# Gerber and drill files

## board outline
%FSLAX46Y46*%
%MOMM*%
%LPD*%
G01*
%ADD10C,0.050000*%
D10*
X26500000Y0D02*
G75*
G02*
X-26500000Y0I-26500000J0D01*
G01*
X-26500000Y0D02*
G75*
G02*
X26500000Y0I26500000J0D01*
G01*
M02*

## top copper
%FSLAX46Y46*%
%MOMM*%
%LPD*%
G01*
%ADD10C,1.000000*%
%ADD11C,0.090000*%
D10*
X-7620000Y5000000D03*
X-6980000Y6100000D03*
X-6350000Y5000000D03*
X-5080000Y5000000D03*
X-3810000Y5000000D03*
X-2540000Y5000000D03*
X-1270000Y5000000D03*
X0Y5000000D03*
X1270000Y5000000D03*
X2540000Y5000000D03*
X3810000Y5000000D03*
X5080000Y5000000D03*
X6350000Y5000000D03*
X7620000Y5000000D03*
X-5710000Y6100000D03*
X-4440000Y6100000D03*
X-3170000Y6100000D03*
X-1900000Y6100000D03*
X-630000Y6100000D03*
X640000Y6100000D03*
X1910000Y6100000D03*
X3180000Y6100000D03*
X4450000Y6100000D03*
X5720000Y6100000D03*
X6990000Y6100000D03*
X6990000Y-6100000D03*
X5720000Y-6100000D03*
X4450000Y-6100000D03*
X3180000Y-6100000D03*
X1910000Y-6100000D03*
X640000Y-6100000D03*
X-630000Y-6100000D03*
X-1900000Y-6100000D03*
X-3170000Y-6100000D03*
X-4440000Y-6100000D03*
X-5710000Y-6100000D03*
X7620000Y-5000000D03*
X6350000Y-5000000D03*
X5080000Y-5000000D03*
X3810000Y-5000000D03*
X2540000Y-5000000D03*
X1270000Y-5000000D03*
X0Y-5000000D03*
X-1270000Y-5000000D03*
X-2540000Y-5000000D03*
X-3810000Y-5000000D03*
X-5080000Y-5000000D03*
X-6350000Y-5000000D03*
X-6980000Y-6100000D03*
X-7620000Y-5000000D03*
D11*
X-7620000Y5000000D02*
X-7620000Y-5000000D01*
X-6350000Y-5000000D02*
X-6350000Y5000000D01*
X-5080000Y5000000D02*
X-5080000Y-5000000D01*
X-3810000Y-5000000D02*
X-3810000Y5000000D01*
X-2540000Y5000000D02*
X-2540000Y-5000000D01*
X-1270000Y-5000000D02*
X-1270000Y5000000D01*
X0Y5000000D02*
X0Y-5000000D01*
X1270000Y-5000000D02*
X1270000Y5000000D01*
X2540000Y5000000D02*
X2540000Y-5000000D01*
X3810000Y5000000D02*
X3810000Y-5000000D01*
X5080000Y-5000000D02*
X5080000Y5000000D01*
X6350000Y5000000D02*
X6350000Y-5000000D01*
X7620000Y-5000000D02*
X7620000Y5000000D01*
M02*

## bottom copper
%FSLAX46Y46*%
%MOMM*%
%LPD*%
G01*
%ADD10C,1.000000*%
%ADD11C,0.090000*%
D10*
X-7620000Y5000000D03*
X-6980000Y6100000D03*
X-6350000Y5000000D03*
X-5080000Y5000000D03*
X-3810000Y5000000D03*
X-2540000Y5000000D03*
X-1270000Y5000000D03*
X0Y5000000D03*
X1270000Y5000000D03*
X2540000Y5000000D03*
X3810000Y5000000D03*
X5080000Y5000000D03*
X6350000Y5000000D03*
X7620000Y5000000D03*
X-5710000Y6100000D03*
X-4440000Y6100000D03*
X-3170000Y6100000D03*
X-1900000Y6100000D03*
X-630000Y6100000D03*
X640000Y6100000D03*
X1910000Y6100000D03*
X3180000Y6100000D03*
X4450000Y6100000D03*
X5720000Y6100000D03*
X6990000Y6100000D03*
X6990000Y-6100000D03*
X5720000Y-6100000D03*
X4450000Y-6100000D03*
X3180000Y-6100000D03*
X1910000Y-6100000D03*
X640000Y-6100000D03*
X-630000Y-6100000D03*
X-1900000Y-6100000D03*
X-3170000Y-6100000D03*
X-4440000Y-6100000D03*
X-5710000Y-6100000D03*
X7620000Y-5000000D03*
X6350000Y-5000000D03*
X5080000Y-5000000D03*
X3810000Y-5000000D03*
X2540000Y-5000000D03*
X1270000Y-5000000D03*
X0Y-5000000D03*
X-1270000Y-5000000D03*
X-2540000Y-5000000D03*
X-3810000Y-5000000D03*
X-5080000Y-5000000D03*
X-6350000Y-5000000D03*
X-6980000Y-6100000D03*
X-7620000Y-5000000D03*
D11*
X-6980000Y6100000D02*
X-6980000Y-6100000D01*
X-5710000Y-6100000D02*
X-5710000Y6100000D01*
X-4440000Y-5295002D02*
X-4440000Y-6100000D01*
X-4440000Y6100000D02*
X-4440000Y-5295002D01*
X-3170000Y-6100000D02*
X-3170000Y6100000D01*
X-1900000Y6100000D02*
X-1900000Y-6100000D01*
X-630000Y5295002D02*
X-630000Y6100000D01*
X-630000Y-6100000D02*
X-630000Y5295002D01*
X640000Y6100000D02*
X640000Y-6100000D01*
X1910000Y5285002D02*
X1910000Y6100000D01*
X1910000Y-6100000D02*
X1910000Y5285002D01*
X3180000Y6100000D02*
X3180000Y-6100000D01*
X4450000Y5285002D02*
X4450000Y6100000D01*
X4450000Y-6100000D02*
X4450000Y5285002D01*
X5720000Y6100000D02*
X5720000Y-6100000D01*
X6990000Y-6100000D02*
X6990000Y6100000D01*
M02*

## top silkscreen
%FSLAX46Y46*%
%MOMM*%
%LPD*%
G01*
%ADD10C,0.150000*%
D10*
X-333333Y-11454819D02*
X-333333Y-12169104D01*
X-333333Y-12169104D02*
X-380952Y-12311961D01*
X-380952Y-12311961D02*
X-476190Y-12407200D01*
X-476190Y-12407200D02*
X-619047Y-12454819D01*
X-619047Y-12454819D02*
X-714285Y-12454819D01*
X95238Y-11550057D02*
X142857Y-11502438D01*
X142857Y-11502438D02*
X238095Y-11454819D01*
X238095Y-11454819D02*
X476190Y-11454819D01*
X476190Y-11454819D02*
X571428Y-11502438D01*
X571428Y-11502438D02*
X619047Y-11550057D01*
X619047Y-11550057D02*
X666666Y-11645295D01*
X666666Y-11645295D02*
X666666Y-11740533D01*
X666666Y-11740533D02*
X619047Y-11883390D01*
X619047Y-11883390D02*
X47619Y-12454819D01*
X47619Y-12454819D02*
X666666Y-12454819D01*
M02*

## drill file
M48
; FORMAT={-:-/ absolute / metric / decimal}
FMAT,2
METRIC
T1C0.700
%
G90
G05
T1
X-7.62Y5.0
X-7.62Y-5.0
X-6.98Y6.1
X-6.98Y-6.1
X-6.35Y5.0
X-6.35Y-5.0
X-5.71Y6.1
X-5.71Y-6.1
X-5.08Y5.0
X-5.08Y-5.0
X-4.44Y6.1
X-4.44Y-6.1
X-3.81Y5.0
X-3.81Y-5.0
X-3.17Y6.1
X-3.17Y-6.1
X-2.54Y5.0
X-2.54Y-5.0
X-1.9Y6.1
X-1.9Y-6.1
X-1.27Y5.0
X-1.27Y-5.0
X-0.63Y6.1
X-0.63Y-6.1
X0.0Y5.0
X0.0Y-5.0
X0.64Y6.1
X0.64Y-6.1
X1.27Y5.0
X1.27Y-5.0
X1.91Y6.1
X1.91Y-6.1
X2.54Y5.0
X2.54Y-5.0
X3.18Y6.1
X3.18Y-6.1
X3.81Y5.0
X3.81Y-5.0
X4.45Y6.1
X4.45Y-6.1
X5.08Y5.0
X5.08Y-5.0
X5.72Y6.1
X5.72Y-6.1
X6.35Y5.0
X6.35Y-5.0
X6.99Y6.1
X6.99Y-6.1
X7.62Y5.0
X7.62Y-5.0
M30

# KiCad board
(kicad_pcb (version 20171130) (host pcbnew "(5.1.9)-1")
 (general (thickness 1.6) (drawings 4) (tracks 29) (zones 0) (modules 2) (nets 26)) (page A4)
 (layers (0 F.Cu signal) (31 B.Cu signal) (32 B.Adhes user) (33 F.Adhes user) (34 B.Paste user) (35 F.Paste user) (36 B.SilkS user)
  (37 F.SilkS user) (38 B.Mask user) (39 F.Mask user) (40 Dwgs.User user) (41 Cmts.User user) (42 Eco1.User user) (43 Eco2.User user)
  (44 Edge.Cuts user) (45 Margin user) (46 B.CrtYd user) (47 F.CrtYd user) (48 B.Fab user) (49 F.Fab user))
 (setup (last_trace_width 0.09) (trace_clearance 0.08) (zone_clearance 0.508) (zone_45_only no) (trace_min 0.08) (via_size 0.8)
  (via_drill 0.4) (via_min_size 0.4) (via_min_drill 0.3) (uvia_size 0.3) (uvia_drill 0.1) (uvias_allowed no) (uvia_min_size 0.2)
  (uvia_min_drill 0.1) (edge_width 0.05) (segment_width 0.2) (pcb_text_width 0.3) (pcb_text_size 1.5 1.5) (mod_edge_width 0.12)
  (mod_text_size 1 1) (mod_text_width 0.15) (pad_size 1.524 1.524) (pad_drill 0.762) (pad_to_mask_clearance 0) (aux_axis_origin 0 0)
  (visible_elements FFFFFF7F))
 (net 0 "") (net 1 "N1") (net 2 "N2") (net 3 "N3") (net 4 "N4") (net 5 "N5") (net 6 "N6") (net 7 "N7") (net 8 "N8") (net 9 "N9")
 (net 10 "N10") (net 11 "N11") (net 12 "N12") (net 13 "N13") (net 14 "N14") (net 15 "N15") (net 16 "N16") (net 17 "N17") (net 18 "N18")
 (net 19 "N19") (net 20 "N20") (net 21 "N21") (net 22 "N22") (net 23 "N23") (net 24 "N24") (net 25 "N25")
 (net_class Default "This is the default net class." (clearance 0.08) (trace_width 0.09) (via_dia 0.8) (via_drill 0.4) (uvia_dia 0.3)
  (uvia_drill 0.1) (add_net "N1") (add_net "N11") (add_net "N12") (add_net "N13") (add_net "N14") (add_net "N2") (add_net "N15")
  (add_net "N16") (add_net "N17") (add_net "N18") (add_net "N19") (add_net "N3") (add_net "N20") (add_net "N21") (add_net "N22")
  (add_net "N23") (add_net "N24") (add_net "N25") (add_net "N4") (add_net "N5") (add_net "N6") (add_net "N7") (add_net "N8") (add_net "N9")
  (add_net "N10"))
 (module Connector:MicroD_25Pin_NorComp (layer B.Cu) (at -7.62 -5)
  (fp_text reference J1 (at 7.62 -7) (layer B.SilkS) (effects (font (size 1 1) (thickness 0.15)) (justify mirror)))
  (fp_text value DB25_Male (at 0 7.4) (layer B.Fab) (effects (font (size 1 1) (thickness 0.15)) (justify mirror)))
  (pad 1 thru_hole circle (at 0 0) (size 1 1) (drill 0.7) (layers *.Cu *.Mask) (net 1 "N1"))
  (pad 14 thru_hole circle (at 0.64 -1.1) (size 1 1) (drill 0.7) (layers *.Cu *.Mask) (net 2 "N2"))
  (pad 2 thru_hole circle (at 1.27 0) (size 1 1) (drill 0.7) (layers *.Cu *.Mask) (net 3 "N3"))
  (pad 3 thru_hole circle (at 2.54 0) (size 1 1) (drill 0.7) (layers *.Cu *.Mask) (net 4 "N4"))
  (pad 4 thru_hole circle (at 3.81 0) (size 1 1) (drill 0.7) (layers *.Cu *.Mask) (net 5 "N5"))
  (pad 5 thru_hole circle (at 5.08 0) (size 1 1) (drill 0.7) (layers *.Cu *.Mask) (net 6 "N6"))
  (pad 6 thru_hole circle (at 6.35 0) (size 1 1) (drill 0.7) (layers *.Cu *.Mask) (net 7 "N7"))
  (pad 7 thru_hole circle (at 7.62 0) (size 1 1) (drill 0.7) (layers *.Cu *.Mask) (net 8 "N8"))
  (pad 8 thru_hole circle (at 8.89 0) (size 1 1) (drill 0.7) (layers *.Cu *.Mask) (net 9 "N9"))
  (pad 9 thru_hole circle (at 10.16 0) (size 1 1) (drill 0.7) (layers *.Cu *.Mask) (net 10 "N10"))
  (pad 10 thru_hole circle (at 11.43 0) (size 1 1) (drill 0.7) (layers *.Cu *.Mask) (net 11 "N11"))
  (pad 11 thru_hole circle (at 12.7 0) (size 1 1) (drill 0.7) (layers *.Cu *.Mask) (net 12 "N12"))
  (pad 12 thru_hole circle (at 13.97 0) (size 1 1) (drill 0.7) (layers *.Cu *.Mask) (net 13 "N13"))
  (pad 13 thru_hole circle (at 15.24 0) (size 1 1) (drill 0.7) (layers *.Cu *.Mask) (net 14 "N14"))
  (pad 15 thru_hole circle (at 1.91 -1.1) (size 1 1) (drill 0.7) (layers *.Cu *.Mask) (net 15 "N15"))
  (pad 16 thru_hole circle (at 3.18 -1.1) (size 1 1) (drill 0.7) (layers *.Cu *.Mask) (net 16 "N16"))
  (pad 17 thru_hole circle (at 4.45 -1.1) (size 1 1) (drill 0.7) (layers *.Cu *.Mask) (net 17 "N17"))
  (pad 18 thru_hole circle (at 5.72 -1.1) (size 1 1) (drill 0.7) (layers *.Cu *.Mask) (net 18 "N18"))
  (pad 19 thru_hole circle (at 6.99 -1.1) (size 1 1) (drill 0.7) (layers *.Cu *.Mask) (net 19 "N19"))
  (pad 20 thru_hole circle (at 8.26 -1.1) (size 1 1) (drill 0.7) (layers *.Cu *.Mask) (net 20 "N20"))
  (pad 21 thru_hole circle (at 9.53 -1.1) (size 1 1) (drill 0.7) (layers *.Cu *.Mask) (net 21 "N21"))
  (pad 22 thru_hole circle (at 10.8 -1.1) (size 1 1) (drill 0.7) (layers *.Cu *.Mask) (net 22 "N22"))
  (pad 23 thru_hole circle (at 12.07 -1.1) (size 1 1) (drill 0.7) (layers *.Cu *.Mask) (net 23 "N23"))
  (pad 24 thru_hole circle (at 13.34 -1.1) (size 1 1) (drill 0.7) (layers *.Cu *.Mask) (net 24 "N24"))
  (pad 25 thru_hole circle (at 14.61 -1.1) (size 1 1) (drill 0.7) (layers *.Cu *.Mask) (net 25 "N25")))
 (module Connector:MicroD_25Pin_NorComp (layer F.Cu) (at -7.62 5)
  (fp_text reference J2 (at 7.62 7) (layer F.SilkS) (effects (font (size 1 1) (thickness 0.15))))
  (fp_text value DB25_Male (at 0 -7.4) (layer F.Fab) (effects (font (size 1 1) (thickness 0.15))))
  (pad 25 thru_hole circle (at 14.61 1.1) (size 1 1) (drill 0.7) (layers *.Cu *.Mask) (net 25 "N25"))
  (pad 24 thru_hole circle (at 13.34 1.1) (size 1 1) (drill 0.7) (layers *.Cu *.Mask) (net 24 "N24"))
  (pad 23 thru_hole circle (at 12.07 1.1) (size 1 1) (drill 0.7) (layers *.Cu *.Mask) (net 23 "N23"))
  (pad 22 thru_hole circle (at 10.8 1.1) (size 1 1) (drill 0.7) (layers *.Cu *.Mask) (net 22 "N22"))
  (pad 21 thru_hole circle (at 9.53 1.1) (size 1 1) (drill 0.7) (layers *.Cu *.Mask) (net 21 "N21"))
  (pad 20 thru_hole circle (at 8.26 1.1) (size 1 1) (drill 0.7) (layers *.Cu *.Mask) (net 20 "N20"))
  (pad 19 thru_hole circle (at 6.99 1.1) (size 1 1) (drill 0.7) (layers *.Cu *.Mask) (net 19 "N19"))
  (pad 18 thru_hole circle (at 5.72 1.1) (size 1 1) (drill 0.7) (layers *.Cu *.Mask) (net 18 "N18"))
  (pad 17 thru_hole circle (at 4.45 1.1) (size 1 1) (drill 0.7) (layers *.Cu *.Mask) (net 17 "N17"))
  (pad 16 thru_hole circle (at 3.18 1.1) (size 1 1) (drill 0.7) (layers *.Cu *.Mask) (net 16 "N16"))
  (pad 15 thru_hole circle (at 1.91 1.1) (size 1 1) (drill 0.7) (layers *.Cu *.Mask) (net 15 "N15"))
  (pad 13 thru_hole circle (at 15.24 0) (size 1 1) (drill 0.7) (layers *.Cu *.Mask) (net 14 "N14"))
  (pad 12 thru_hole circle (at 13.97 0) (size 1 1) (drill 0.7) (layers *.Cu *.Mask) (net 13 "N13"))
  (pad 11 thru_hole circle (at 12.7 0) (size 1 1) (drill 0.7) (layers *.Cu *.Mask) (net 12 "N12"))
  (pad 10 thru_hole circle (at 11.43 0) (size 1 1) (drill 0.7) (layers *.Cu *.Mask) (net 11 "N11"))
  (pad 9 thru_hole circle (at 10.16 0) (size 1 1) (drill 0.7) (layers *.Cu *.Mask) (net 10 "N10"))
  (pad 8 thru_hole circle (at 8.89 0) (size 1 1) (drill 0.7) (layers *.Cu *.Mask) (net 9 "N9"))
  (pad 7 thru_hole circle (at 7.62 0) (size 1 1) (drill 0.7) (layers *.Cu *.Mask) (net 8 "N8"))
  (pad 6 thru_hole circle (at 6.35 0) (size 1 1) (drill 0.7) (layers *.Cu *.Mask) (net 7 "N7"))
  (pad 5 thru_hole circle (at 5.08 0) (size 1 1) (drill 0.7) (layers *.Cu *.Mask) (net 6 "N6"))
  (pad 4 thru_hole circle (at 3.81 0) (size 1 1) (drill 0.7) (layers *.Cu *.Mask) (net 5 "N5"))
  (pad 3 thru_hole circle (at 2.54 0) (size 1 1) (drill 0.7) (layers *.Cu *.Mask) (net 4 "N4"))
  (pad 2 thru_hole circle (at 1.27 0) (size 1 1) (drill 0.7) (layers *.Cu *.Mask) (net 3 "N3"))
  (pad 14 thru_hole circle (at 0.64 1.1) (size 1 1) (drill 0.7) (layers *.Cu *.Mask) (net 2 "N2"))
  (pad 1 thru_hole circle (at 0 0) (size 1 1) (drill 0.7) (layers *.Cu *.Mask) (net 1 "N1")))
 (gr_circle (center 0 0) (end 26.5 0) (layer Edge.Cuts) (width 0.05))
 (segment (start -7.62 -5) (end -7.62 5) (width 0.09) (layer F.Cu) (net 1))
 (segment (start -6.98 -6.1) (end -6.98 6.1) (width 0.09) (layer B.Cu) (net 2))
 (segment (start -6.35 5) (end -6.35 -5) (width 0.09) (layer F.Cu) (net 3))
 (segment (start -5.08 -5) (end -5.08 5) (width 0.09) (layer F.Cu) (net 4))
 (segment (start -3.81 5) (end -3.81 -5) (width 0.09) (layer F.Cu) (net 5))
 (segment (start -2.54 -5) (end -2.54 5) (width 0.09) (layer F.Cu) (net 6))
 (segment (start -1.27 5) (end -1.27 -5) (width 0.09) (layer F.Cu) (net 7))
 (segment (start 0 -5) (end 0 5) (width 0.09) (layer F.Cu) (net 8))
 (segment (start 1.27 5) (end 1.27 -5) (width 0.09) (layer F.Cu) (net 9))
 (segment (start 2.54 -5) (end 2.54 5) (width 0.09) (layer F.Cu) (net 10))
 (segment (start 3.81 -5) (end 3.81 5) (width 0.09) (layer F.Cu) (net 11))
 (segment (start 5.08 5) (end 5.08 -5) (width 0.09) (layer F.Cu) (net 12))
 (segment (start 6.35 -5) (end 6.35 5) (width 0.09) (layer F.Cu) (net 13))
 (segment (start 7.62 5) (end 7.62 -5) (width 0.09) (layer F.Cu) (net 14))
 (segment (start -5.71 6.1) (end -5.71 -6.1) (width 0.09) (layer B.Cu) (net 15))
 (segment (start -4.44 5.295002) (end -4.44 6.1) (width 0.09) (layer B.Cu) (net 16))
 (segment (start -4.44 -6.1) (end -4.44 5.295002) (width 0.09) (layer B.Cu) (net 16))
 (segment (start -3.17 6.1) (end -3.17 -6.1) (width 0.09) (layer B.Cu) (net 17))
 (segment (start -1.9 -6.1) (end -1.9 6.1) (width 0.09) (layer B.Cu) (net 18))
 (segment (start -0.63 -5.295002) (end -0.63 -6.1) (width 0.09) (layer B.Cu) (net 19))
 (segment (start -0.63 6.1) (end -0.63 -5.295002) (width 0.09) (layer B.Cu) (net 19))
 (segment (start 0.64 -6.1) (end 0.64 6.1) (width 0.09) (layer B.Cu) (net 20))
 (segment (start 1.91 -5.285002) (end 1.91 -6.1) (width 0.09) (layer B.Cu) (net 21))
 (segment (start 1.91 6.1) (end 1.91 -5.285002) (width 0.09) (layer B.Cu) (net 21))
 (segment (start 3.18 -6.1) (end 3.18 6.1) (width 0.09) (layer B.Cu) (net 22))
 (segment (start 4.45 -5.285002) (end 4.45 -6.1) (width 0.09) (layer B.Cu) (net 23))
 (segment (start 4.45 6.1) (end 4.45 -5.285002) (width 0.09) (layer B.Cu) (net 23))
 (segment (start 5.72 -6.1) (end 5.72 6.1) (width 0.09) (layer B.Cu) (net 24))
 (segment (start 6.99 6.1) (end 6.99 -6.1) (width 0.09) (layer B.Cu) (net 25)))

